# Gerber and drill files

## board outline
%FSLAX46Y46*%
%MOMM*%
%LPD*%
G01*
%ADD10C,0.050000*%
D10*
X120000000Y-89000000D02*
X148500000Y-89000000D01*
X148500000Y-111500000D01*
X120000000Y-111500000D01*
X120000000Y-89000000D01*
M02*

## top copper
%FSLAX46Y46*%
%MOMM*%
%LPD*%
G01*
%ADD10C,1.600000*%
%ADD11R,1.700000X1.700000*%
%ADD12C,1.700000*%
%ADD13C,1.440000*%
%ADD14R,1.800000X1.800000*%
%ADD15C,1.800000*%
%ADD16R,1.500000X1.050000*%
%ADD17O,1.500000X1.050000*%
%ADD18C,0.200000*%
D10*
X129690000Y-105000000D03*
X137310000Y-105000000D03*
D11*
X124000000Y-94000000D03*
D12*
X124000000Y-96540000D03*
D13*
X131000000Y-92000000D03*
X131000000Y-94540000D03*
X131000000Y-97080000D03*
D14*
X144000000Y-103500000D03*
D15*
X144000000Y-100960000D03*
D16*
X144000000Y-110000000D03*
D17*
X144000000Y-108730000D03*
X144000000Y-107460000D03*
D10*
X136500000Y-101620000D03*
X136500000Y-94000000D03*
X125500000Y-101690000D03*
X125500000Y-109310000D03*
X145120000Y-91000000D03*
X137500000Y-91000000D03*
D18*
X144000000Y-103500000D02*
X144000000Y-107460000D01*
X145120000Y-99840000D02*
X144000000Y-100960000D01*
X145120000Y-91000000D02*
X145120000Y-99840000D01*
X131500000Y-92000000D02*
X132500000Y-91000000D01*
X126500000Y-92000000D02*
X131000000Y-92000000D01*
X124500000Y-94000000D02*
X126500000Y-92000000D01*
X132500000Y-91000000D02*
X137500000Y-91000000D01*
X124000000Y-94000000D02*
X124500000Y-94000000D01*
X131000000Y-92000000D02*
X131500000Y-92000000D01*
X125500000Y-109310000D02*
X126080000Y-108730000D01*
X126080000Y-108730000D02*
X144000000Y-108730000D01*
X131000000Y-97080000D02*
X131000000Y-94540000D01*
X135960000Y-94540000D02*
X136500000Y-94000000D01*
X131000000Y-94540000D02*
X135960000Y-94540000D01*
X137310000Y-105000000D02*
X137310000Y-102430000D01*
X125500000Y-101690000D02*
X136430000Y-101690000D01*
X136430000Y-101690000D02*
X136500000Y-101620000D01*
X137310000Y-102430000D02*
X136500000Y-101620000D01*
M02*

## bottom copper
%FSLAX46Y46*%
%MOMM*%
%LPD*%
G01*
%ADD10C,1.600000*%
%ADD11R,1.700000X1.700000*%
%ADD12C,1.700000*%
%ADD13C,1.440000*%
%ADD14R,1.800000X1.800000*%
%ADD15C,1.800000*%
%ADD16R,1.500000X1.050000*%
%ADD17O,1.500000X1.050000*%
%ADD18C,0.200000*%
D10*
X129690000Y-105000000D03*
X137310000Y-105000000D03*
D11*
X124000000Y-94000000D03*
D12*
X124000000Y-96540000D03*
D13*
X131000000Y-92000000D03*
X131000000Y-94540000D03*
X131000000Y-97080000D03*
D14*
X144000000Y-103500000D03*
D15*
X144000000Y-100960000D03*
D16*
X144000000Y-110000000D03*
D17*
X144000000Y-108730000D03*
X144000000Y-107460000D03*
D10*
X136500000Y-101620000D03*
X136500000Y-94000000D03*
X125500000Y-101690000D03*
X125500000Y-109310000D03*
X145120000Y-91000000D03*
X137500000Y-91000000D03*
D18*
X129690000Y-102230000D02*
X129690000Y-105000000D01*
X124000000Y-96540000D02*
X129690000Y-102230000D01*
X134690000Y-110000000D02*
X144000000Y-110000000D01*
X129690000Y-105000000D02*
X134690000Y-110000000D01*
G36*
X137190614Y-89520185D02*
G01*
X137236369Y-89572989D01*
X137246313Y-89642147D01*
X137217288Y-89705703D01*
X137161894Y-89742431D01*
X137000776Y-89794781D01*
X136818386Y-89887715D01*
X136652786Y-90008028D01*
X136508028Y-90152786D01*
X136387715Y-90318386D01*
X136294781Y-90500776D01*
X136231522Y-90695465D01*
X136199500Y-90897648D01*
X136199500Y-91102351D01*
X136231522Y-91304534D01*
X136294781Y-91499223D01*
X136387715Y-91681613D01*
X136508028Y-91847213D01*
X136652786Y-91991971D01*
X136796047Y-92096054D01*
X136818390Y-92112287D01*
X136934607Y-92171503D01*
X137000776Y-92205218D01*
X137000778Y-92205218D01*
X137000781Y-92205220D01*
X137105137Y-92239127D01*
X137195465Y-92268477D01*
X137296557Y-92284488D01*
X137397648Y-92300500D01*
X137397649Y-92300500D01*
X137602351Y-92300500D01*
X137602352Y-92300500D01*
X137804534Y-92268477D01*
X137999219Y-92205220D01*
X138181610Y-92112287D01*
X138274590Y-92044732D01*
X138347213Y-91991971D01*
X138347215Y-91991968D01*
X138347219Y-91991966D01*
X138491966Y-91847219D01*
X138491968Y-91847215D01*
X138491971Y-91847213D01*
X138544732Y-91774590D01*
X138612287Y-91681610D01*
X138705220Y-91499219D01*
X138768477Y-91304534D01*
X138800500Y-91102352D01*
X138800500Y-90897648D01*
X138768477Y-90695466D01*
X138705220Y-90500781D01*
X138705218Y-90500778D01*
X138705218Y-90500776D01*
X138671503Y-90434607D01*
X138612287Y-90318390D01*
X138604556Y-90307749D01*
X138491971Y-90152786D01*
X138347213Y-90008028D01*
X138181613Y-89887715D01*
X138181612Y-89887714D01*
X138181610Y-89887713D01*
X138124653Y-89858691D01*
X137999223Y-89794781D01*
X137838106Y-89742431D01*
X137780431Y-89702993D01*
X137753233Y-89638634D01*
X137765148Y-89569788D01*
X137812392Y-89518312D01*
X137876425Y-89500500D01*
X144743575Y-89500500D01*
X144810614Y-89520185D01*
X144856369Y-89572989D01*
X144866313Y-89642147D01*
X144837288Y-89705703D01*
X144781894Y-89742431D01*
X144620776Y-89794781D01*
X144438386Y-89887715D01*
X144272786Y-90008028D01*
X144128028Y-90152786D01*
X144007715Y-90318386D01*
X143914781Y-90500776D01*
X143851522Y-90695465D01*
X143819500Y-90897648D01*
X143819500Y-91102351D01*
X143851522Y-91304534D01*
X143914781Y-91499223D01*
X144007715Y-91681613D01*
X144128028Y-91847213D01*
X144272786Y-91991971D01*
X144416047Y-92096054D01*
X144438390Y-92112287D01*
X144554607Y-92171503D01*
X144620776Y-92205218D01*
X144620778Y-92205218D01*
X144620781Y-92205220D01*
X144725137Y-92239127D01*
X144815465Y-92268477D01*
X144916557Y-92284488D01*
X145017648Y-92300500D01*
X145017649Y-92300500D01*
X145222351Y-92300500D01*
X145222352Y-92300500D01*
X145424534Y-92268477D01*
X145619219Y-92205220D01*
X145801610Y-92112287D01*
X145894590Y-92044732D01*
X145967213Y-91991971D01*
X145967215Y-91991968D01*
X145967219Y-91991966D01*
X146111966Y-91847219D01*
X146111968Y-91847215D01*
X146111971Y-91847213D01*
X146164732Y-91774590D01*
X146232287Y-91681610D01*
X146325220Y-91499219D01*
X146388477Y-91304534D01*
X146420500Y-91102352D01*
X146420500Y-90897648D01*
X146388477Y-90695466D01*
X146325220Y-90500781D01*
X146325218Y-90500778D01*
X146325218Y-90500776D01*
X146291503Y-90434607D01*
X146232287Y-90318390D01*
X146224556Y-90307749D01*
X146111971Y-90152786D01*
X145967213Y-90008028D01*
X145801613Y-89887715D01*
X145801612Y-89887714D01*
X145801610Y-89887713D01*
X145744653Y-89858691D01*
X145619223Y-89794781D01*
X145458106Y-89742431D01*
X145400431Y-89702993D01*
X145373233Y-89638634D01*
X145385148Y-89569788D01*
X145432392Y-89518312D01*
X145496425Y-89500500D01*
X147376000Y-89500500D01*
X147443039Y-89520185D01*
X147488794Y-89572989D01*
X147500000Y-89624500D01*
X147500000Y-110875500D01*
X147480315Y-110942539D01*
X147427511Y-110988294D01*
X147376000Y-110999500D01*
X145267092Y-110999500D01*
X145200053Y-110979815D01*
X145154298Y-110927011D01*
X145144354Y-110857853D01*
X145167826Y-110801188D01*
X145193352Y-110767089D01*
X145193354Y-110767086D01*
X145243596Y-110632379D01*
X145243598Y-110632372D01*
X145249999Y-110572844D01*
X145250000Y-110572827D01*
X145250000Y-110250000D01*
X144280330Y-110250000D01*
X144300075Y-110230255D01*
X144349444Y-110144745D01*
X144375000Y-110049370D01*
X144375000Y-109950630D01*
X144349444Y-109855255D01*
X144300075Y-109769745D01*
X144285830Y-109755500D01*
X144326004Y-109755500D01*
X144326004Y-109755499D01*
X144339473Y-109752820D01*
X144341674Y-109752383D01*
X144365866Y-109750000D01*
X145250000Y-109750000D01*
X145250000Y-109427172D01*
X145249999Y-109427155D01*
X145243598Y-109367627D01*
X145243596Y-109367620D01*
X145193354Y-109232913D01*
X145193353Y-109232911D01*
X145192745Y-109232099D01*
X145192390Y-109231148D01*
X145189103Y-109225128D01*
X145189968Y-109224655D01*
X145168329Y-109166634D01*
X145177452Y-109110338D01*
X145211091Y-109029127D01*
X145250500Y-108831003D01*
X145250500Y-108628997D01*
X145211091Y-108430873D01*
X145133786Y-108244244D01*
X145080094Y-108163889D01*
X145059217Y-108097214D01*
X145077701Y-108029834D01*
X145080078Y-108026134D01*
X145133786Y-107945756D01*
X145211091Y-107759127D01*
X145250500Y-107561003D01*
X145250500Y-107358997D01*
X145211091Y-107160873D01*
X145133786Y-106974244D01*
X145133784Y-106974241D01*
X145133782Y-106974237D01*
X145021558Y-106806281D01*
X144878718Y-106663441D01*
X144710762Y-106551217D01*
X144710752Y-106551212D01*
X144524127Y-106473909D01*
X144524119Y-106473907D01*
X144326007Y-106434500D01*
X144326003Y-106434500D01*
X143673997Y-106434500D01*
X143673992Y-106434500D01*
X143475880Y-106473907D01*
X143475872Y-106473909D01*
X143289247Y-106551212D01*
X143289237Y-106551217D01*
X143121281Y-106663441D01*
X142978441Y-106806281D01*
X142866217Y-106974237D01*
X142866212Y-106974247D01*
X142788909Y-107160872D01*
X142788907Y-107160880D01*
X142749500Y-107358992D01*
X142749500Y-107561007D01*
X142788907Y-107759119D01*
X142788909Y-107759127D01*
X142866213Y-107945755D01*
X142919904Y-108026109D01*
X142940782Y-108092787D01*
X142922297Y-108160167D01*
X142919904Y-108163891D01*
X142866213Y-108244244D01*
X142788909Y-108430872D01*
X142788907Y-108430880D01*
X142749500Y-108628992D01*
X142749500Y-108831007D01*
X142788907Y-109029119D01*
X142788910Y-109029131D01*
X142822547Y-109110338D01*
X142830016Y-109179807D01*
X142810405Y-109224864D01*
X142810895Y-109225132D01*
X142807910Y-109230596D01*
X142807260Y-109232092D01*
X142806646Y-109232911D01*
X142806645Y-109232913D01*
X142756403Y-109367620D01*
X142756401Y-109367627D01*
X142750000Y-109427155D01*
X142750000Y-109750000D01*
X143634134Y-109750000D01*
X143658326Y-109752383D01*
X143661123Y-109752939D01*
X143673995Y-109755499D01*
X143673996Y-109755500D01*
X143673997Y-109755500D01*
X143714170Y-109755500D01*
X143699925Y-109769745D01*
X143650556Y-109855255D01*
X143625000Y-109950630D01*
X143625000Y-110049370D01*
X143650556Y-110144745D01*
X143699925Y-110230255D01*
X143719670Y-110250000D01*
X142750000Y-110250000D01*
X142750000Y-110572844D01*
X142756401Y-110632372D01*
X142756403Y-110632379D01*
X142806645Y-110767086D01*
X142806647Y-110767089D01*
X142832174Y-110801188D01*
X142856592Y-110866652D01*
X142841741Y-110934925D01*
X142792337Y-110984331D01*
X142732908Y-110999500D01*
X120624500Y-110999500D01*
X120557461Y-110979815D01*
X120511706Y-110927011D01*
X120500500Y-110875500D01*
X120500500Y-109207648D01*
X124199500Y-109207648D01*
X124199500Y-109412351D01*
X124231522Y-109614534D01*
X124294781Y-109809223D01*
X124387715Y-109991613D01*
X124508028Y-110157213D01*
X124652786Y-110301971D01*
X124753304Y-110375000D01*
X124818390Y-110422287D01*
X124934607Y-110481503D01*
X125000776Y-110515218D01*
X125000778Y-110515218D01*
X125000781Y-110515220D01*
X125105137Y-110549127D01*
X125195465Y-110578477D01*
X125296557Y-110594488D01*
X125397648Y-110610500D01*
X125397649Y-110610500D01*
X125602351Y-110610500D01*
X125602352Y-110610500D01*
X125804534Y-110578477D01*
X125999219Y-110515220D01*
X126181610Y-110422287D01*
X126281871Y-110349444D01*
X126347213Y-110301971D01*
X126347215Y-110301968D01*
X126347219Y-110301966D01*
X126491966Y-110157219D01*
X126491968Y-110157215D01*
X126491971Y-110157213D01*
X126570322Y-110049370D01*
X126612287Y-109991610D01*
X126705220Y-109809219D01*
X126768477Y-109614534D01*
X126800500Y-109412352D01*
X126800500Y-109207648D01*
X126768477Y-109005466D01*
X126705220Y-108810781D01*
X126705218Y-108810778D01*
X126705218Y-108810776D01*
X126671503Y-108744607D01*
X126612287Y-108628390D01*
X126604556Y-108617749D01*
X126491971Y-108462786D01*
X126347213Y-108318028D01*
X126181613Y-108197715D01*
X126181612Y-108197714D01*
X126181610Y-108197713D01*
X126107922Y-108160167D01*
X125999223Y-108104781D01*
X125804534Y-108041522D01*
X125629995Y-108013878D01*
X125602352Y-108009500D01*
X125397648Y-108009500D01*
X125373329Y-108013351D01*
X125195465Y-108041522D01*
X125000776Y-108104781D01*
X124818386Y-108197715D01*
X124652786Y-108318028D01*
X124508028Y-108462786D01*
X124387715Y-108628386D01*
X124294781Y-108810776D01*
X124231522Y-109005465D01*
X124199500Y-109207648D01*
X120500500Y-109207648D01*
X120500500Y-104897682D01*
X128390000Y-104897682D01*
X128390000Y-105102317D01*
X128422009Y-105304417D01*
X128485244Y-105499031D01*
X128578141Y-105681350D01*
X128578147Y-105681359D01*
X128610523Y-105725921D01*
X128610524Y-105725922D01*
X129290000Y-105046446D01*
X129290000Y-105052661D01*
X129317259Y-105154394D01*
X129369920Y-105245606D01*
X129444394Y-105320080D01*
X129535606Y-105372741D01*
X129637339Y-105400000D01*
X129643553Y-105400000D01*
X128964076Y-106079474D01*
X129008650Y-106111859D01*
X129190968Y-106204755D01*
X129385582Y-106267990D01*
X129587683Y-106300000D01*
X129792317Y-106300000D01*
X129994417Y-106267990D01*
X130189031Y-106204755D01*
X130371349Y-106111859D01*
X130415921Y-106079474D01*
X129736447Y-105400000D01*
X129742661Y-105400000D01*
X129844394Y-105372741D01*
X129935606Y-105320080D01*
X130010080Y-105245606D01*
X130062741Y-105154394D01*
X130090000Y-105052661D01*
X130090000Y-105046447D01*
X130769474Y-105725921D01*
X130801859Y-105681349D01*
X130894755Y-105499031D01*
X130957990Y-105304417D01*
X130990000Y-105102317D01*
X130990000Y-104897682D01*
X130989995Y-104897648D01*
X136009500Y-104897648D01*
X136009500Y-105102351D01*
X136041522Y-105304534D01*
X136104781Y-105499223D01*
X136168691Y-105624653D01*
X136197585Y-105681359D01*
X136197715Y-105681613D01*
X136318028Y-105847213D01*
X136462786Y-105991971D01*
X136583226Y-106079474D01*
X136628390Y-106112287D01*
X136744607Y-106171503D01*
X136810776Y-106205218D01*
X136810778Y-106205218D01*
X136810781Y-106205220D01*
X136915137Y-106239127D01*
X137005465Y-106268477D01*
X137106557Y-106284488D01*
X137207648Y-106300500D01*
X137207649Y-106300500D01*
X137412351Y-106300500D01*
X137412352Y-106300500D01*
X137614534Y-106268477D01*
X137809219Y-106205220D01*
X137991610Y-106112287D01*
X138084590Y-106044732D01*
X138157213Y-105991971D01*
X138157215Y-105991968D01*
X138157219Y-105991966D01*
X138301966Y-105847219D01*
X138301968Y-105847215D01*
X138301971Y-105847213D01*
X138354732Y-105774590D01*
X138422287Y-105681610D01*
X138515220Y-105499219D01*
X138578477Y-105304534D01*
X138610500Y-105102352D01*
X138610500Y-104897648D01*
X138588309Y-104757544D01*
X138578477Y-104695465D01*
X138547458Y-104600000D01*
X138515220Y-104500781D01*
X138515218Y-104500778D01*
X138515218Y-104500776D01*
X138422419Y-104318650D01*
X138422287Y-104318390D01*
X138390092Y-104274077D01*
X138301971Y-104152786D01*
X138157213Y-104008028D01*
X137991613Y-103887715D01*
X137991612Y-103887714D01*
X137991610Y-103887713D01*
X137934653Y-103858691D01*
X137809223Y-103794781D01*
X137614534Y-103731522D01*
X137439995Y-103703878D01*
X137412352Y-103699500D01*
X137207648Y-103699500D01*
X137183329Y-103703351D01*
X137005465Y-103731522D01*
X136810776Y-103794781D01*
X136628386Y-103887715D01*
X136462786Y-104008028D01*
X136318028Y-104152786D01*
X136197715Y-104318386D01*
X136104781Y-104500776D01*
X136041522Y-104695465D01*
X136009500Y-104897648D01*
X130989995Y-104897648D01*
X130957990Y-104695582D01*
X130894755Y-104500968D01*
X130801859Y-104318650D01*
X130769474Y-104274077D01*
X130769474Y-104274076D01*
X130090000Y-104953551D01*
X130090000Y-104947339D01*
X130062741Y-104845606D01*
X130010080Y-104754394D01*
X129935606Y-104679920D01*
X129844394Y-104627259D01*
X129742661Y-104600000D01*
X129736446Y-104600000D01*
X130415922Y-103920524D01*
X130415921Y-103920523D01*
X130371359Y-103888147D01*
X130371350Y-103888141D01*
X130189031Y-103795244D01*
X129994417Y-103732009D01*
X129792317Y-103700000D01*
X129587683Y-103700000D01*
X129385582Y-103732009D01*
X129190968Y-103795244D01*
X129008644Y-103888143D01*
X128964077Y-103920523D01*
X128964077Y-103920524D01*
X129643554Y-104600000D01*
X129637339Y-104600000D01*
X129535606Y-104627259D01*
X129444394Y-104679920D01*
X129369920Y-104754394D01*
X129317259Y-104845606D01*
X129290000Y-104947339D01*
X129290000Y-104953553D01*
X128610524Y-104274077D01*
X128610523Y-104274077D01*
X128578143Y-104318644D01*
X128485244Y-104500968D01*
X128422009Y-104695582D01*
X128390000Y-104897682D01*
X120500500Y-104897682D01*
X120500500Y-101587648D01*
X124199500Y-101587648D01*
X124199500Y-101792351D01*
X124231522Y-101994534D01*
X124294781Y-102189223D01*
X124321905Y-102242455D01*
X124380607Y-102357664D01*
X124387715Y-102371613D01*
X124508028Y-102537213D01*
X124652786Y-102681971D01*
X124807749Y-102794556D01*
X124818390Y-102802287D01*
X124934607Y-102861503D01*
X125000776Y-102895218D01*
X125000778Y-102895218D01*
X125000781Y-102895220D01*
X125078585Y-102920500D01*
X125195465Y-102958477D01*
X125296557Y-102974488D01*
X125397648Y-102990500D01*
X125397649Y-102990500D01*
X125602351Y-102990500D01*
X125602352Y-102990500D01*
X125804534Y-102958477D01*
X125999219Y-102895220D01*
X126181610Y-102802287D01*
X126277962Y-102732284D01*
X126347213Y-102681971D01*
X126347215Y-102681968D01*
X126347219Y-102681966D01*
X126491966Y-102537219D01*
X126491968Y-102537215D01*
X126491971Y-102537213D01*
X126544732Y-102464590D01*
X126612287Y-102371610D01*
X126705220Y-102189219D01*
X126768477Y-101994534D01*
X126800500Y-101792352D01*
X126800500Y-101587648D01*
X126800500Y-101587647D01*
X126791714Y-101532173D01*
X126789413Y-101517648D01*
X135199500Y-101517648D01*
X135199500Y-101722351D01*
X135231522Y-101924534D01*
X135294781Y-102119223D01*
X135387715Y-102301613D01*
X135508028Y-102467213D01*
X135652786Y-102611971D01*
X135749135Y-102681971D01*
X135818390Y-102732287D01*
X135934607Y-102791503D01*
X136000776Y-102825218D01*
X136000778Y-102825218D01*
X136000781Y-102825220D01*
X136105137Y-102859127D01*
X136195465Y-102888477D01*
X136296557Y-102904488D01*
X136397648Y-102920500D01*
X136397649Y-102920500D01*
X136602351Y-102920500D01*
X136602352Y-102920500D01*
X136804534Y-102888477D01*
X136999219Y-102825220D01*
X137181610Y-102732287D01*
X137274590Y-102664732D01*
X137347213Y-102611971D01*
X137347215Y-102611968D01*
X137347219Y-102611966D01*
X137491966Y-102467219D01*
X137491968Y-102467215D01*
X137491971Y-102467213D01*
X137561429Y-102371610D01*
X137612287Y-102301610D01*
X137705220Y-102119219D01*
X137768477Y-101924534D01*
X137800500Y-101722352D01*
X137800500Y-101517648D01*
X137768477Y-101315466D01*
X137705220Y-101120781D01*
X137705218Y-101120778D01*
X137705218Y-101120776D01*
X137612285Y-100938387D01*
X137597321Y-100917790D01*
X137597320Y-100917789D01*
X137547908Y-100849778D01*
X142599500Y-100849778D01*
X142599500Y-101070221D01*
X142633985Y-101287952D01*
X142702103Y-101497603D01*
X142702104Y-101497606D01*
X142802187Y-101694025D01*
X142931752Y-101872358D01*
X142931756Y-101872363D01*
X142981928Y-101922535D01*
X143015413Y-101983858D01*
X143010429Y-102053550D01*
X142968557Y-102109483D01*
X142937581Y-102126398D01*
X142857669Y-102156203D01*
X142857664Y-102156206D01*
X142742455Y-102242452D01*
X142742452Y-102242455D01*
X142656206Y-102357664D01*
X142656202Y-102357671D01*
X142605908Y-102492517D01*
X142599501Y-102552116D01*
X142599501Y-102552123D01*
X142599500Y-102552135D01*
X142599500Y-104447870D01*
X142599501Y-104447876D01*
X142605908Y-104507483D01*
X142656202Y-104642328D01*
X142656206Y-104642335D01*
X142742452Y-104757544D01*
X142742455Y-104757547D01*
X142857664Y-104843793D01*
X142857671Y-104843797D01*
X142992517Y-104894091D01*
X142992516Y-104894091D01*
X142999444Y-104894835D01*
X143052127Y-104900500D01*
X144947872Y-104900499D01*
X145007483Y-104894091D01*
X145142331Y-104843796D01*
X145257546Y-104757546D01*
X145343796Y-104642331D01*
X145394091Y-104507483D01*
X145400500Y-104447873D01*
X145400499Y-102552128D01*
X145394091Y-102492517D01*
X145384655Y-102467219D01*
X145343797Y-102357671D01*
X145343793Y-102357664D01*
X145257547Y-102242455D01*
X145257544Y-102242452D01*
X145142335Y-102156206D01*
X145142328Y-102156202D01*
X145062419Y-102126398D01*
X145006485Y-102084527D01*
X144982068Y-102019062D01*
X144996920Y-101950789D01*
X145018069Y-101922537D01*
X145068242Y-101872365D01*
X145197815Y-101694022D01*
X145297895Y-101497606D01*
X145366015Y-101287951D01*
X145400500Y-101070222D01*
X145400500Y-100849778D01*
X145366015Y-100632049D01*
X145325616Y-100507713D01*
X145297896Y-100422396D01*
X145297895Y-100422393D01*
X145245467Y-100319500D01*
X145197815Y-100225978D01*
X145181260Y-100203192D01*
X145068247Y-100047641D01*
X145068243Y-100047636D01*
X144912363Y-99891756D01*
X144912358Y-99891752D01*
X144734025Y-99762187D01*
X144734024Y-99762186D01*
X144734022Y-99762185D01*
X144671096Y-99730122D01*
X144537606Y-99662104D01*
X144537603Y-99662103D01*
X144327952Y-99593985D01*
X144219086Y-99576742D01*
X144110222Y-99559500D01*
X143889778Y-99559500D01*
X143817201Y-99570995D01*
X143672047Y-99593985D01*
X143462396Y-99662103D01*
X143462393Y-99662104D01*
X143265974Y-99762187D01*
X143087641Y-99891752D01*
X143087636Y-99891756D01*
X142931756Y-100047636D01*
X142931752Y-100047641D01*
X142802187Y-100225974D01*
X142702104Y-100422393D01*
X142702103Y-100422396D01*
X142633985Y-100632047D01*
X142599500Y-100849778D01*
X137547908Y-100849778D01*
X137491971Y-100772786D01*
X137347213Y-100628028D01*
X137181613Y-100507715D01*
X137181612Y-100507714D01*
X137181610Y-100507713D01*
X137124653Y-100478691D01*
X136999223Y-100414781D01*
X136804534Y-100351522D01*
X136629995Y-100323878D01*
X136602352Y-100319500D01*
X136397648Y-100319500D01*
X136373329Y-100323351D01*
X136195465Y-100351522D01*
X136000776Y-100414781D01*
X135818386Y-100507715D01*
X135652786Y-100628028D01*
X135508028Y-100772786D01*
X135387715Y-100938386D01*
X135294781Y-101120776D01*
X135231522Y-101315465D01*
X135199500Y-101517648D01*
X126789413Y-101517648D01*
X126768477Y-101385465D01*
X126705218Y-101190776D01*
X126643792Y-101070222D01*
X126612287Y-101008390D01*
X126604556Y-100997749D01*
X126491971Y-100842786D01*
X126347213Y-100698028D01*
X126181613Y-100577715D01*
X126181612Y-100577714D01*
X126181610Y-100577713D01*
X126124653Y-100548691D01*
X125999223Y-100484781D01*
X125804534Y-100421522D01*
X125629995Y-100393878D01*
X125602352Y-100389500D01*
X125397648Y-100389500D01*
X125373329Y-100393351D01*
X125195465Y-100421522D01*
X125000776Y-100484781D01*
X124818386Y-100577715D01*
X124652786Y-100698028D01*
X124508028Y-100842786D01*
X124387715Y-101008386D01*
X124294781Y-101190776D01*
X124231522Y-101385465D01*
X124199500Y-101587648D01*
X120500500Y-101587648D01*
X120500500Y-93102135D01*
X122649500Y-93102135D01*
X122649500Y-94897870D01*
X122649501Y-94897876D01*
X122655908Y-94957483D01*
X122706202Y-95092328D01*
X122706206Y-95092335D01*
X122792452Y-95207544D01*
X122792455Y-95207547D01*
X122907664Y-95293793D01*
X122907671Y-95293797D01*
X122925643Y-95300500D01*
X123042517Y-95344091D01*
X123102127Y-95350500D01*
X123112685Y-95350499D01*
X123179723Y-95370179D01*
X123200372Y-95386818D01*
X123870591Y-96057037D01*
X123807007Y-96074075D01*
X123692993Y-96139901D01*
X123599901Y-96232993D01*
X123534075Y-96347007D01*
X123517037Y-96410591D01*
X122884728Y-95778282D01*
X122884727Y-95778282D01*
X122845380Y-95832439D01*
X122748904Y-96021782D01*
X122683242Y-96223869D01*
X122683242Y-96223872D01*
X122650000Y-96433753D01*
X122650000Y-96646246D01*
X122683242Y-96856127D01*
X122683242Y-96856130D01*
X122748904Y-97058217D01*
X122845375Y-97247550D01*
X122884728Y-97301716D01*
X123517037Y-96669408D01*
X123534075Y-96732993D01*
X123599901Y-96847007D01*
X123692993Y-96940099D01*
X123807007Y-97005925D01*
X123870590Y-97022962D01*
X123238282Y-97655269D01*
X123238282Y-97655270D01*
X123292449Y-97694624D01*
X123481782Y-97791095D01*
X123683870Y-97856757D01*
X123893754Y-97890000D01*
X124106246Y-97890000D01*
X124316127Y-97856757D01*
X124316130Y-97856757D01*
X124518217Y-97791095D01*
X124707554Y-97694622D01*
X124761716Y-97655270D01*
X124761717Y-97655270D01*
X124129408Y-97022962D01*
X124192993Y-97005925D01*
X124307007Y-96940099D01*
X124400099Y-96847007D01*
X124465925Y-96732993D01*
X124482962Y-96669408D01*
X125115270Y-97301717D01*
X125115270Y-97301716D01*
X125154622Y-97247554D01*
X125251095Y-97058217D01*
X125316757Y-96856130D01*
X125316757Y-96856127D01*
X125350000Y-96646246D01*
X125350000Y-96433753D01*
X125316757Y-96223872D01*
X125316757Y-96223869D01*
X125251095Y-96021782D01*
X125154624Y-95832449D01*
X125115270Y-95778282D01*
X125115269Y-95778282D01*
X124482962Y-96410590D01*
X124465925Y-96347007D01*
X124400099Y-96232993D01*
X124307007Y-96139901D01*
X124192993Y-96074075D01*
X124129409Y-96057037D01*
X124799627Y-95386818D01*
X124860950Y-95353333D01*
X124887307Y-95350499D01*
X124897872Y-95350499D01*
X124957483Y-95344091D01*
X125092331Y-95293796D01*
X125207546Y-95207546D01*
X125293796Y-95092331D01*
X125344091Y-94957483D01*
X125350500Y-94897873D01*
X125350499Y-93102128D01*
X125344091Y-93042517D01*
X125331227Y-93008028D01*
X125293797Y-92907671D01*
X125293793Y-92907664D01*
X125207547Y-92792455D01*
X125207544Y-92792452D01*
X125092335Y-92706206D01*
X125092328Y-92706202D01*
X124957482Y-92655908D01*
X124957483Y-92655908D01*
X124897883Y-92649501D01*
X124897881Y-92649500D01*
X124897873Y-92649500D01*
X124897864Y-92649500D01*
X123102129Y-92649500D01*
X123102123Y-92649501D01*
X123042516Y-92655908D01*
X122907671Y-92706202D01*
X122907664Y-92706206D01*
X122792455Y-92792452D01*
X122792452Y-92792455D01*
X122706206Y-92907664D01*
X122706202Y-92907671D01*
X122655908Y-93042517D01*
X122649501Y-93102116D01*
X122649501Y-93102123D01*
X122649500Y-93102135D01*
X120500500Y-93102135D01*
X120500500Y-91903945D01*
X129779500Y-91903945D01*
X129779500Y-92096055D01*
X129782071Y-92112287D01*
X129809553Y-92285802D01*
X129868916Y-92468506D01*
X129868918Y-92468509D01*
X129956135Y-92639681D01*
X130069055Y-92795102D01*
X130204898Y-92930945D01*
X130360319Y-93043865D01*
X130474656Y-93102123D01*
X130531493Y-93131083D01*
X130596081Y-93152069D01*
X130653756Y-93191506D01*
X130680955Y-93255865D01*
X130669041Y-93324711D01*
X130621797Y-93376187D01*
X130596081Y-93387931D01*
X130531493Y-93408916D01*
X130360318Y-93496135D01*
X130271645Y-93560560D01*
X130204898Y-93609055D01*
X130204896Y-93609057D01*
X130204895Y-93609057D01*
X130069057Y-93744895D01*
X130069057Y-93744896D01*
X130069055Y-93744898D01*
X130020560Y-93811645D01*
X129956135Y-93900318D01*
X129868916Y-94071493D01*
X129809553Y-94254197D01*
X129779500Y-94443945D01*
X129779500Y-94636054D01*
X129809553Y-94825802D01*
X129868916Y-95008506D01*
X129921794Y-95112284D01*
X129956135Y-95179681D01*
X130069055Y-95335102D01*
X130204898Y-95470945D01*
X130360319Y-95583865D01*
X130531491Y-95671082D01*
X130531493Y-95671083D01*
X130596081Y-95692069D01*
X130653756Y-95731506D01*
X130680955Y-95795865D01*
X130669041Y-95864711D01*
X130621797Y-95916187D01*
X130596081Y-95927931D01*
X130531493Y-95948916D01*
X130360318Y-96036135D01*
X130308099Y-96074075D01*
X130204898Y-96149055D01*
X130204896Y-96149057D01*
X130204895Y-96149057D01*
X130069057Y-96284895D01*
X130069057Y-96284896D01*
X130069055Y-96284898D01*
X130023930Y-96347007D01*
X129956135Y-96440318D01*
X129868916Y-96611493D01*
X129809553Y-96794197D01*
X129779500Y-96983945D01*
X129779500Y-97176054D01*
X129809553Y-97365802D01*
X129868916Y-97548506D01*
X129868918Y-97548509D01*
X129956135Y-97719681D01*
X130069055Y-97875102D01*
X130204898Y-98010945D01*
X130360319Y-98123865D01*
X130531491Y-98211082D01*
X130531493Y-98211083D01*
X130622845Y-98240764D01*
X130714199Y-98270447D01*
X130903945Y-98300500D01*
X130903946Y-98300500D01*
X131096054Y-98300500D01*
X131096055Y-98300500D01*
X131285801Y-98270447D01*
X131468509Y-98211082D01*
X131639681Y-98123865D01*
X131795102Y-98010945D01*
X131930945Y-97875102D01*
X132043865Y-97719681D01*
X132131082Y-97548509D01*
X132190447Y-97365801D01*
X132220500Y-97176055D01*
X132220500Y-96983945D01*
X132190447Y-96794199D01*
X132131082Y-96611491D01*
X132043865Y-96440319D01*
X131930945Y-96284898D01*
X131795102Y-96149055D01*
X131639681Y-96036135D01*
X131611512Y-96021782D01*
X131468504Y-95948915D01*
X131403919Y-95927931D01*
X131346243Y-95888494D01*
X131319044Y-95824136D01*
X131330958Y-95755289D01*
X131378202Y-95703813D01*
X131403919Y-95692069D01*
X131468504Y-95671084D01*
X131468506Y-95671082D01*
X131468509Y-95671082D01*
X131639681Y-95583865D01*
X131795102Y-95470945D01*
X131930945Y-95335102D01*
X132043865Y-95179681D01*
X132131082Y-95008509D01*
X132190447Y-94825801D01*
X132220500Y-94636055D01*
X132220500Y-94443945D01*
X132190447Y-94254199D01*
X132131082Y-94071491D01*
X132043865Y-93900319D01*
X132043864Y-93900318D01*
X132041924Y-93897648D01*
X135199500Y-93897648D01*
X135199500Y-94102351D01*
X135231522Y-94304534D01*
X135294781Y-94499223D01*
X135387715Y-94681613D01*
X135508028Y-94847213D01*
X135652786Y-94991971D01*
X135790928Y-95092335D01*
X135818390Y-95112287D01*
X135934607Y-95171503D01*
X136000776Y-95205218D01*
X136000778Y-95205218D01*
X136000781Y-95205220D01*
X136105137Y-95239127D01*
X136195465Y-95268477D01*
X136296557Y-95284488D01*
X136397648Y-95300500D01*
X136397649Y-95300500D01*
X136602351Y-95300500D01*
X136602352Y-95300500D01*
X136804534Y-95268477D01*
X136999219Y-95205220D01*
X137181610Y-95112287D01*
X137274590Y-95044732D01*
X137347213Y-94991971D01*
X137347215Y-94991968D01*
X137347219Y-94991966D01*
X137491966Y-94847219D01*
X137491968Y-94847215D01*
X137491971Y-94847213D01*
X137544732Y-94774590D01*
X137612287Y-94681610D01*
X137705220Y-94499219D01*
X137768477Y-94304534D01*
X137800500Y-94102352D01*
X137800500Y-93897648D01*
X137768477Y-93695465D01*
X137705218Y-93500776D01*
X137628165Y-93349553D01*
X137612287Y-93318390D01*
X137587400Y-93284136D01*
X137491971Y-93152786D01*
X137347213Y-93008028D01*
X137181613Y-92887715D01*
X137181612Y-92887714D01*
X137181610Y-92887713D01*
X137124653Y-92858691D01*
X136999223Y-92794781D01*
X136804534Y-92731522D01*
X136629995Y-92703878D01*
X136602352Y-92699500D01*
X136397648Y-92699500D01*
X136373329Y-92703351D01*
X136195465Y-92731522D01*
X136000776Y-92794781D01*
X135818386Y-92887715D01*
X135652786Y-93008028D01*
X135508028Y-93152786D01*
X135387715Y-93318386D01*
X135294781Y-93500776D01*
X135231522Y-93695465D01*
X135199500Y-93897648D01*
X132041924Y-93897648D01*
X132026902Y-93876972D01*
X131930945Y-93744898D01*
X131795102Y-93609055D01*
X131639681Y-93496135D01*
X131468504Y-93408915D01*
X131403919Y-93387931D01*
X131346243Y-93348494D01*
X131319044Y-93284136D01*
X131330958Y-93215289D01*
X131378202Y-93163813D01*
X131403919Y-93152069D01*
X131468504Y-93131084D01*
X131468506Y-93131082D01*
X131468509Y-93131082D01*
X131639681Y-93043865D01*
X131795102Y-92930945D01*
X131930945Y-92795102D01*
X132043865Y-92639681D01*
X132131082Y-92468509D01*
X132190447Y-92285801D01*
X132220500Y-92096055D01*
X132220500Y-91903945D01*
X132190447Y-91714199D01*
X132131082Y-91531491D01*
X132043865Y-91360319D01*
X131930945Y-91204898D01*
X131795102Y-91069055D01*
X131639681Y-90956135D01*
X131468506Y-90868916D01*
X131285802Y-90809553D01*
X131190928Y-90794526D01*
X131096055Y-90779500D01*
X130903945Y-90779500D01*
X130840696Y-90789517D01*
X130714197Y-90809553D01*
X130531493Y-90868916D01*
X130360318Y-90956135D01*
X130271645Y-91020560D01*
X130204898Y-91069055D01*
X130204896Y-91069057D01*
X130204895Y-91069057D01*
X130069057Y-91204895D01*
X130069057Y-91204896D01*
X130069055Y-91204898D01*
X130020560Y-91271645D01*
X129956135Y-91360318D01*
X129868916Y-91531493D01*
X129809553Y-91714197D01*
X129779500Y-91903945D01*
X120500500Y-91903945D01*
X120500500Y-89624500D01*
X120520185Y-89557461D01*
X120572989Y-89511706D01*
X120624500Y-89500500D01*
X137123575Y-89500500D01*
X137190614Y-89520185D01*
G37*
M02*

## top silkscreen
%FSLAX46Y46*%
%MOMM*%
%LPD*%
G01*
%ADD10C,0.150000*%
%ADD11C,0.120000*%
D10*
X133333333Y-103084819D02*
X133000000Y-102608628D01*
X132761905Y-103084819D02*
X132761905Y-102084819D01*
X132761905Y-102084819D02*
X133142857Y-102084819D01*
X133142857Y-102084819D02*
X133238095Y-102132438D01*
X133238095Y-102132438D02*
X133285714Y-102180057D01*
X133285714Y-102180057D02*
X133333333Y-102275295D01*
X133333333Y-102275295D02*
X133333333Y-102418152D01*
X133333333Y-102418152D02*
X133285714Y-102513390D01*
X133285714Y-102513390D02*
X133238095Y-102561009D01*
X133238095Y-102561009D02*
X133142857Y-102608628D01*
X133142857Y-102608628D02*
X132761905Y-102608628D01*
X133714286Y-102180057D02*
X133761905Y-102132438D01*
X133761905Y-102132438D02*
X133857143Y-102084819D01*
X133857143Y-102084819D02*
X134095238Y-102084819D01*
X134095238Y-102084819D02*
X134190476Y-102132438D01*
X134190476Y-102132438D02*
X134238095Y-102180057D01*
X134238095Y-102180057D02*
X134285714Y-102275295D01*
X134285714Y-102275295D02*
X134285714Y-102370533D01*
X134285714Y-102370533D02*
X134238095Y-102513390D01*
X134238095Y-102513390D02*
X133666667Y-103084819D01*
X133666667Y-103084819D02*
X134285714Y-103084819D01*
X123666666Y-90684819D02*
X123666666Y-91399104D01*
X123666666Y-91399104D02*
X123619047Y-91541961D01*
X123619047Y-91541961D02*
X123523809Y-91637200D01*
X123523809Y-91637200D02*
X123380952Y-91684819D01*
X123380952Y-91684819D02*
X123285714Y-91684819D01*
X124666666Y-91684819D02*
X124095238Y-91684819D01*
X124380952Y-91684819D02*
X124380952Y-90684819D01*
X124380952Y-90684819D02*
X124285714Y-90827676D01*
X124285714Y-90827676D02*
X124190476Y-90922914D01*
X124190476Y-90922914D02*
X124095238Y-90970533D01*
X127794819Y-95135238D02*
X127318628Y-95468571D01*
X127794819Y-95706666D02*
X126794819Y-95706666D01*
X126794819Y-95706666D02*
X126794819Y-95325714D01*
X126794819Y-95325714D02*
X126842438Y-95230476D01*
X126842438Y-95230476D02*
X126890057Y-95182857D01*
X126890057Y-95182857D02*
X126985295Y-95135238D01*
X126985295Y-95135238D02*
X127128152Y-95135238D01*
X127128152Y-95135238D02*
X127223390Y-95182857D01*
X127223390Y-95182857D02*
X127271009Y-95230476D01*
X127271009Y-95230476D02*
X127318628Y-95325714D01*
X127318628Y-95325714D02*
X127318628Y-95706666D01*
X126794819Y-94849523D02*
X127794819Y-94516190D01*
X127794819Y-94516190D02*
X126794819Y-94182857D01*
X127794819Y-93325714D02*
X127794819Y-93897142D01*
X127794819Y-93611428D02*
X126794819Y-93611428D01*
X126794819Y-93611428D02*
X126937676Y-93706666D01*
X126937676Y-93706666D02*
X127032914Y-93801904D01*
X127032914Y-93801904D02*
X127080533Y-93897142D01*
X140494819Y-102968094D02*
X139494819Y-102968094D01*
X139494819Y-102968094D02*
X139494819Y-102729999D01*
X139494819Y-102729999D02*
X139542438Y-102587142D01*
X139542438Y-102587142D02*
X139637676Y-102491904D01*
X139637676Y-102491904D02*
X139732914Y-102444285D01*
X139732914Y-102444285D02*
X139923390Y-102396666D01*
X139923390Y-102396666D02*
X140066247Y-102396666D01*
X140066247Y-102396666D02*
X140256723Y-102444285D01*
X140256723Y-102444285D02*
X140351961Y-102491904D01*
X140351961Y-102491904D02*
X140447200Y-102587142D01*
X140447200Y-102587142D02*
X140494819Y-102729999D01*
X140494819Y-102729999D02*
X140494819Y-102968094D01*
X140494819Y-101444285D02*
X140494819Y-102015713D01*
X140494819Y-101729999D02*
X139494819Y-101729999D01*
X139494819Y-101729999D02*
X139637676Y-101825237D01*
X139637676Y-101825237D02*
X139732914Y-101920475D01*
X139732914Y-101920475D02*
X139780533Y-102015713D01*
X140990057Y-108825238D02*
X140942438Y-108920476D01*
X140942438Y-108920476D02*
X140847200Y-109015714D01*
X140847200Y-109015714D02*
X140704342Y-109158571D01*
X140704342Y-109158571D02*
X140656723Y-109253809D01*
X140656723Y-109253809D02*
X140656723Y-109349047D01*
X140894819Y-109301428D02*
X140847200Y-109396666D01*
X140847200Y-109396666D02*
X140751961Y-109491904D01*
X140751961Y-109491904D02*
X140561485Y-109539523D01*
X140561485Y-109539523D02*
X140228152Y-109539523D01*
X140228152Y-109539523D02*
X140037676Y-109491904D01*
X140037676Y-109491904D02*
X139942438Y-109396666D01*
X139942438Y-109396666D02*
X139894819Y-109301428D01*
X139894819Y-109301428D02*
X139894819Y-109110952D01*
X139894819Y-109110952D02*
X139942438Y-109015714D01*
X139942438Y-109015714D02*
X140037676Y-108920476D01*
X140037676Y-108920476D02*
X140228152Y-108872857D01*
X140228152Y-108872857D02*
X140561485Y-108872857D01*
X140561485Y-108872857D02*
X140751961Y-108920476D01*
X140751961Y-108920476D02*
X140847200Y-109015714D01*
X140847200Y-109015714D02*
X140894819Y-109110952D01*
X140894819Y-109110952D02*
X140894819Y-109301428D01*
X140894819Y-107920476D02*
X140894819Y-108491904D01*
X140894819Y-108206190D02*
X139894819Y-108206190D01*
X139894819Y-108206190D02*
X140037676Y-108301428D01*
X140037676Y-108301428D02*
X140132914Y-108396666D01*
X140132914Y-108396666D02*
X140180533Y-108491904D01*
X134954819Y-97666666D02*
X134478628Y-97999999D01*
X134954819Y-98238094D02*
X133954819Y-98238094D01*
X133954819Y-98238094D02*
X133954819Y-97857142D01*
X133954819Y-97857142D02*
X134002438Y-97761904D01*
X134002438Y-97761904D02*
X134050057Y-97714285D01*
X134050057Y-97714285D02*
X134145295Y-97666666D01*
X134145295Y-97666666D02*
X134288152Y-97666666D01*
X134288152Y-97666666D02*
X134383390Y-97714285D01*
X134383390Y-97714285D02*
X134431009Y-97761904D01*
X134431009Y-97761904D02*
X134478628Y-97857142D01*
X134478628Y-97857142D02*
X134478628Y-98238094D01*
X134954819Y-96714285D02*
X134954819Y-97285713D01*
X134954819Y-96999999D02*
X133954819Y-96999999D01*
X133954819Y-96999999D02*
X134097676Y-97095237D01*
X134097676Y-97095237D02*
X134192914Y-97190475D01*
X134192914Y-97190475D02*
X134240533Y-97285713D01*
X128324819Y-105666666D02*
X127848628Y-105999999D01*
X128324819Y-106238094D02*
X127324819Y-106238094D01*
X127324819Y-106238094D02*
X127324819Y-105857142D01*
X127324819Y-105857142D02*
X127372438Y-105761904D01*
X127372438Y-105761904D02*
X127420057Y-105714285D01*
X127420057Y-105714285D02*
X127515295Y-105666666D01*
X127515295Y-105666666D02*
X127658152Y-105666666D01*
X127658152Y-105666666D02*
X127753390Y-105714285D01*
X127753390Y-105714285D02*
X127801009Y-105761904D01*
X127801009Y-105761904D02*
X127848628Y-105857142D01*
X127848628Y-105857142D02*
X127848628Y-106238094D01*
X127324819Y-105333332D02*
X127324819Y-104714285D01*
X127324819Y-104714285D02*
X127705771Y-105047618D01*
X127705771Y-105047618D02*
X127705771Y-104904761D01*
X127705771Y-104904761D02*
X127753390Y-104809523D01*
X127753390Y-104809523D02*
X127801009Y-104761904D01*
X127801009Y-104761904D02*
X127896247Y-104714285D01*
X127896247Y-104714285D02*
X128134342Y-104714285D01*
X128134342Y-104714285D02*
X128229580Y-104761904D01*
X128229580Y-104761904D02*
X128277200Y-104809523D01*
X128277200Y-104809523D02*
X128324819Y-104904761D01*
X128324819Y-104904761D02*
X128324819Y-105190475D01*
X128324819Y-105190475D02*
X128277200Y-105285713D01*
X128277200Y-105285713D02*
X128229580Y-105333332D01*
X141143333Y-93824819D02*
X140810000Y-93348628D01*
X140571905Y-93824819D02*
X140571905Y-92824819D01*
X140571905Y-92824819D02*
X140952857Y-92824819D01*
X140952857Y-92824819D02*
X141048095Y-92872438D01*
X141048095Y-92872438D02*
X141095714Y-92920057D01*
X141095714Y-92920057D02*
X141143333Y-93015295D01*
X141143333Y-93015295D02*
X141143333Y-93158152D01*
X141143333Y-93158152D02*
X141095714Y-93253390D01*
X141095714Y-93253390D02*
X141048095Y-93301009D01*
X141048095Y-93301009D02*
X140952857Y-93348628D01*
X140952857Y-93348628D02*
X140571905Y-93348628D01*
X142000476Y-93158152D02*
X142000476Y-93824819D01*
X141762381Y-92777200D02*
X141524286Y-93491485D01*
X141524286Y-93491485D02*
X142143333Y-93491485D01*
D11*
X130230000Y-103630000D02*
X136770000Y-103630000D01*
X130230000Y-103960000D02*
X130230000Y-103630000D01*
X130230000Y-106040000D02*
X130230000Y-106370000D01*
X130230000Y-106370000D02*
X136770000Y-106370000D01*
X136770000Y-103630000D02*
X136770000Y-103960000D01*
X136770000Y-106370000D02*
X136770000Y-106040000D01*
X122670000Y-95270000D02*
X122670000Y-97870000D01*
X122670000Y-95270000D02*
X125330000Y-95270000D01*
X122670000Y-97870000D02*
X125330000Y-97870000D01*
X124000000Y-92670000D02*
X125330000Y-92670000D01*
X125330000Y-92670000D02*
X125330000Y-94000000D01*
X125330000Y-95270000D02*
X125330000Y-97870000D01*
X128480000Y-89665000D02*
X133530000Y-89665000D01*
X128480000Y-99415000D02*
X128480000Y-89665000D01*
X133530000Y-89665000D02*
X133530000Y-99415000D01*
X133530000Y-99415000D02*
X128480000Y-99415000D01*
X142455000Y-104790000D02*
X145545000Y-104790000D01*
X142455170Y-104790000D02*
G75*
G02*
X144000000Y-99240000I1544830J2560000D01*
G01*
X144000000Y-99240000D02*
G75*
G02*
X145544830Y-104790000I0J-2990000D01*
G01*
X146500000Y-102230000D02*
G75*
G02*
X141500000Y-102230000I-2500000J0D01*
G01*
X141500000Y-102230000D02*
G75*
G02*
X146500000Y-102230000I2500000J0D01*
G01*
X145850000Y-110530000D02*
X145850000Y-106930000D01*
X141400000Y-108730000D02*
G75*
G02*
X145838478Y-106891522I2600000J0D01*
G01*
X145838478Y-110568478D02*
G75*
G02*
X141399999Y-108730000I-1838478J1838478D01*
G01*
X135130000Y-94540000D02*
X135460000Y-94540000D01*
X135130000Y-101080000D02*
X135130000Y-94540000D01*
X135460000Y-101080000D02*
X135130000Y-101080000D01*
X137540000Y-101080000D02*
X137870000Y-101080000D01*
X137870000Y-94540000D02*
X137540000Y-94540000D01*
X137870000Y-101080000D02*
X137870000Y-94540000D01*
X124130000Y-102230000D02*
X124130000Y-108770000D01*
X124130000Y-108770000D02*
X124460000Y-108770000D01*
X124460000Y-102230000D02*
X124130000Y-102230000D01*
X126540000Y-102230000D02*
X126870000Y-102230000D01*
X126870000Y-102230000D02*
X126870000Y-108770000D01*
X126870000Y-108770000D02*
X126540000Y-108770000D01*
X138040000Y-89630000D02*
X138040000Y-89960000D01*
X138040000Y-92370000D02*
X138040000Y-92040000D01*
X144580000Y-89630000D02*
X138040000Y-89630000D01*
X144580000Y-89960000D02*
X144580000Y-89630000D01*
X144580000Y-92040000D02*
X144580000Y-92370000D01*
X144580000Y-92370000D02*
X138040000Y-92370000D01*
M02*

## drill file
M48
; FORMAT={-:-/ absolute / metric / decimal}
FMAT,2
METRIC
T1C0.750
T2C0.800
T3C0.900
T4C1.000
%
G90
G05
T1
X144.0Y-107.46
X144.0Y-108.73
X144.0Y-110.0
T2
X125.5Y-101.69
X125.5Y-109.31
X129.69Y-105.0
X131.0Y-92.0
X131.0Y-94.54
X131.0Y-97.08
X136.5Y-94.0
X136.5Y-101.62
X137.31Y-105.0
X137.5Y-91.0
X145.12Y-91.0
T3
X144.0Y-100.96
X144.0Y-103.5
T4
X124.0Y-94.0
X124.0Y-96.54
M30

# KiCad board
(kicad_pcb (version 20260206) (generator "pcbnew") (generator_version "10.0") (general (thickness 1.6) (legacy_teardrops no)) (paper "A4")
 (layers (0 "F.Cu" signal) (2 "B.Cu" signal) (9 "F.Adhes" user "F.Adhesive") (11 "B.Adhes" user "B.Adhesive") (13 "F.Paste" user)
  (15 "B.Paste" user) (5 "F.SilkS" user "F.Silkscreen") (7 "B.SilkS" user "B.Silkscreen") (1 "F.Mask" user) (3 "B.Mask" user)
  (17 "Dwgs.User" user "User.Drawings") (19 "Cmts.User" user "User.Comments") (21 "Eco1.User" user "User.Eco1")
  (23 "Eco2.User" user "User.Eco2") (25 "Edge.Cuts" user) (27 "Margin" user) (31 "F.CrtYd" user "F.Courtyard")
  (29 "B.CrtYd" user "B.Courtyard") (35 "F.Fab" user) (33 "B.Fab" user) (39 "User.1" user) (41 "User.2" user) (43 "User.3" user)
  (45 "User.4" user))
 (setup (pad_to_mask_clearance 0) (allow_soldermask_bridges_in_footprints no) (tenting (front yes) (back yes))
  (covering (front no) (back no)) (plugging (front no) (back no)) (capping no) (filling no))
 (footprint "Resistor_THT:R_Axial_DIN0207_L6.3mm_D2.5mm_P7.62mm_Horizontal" (layer "F.Cu") (at 129.69 105)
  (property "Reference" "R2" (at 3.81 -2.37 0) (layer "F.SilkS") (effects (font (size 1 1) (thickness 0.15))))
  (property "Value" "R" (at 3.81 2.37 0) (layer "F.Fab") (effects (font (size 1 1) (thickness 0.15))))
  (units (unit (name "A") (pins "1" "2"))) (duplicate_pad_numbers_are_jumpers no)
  (fp_line (start 0.54 -1.37) (end 7.08 -1.37) (stroke (width 0.12) (type solid)) (layer "F.SilkS"))
  (fp_line (start 0.54 -1.04) (end 0.54 -1.37) (stroke (width 0.12) (type solid)) (layer "F.SilkS"))
  (fp_line (start 0.54 1.04) (end 0.54 1.37) (stroke (width 0.12) (type solid)) (layer "F.SilkS"))
  (fp_line (start 0.54 1.37) (end 7.08 1.37) (stroke (width 0.12) (type solid)) (layer "F.SilkS"))
  (fp_line (start 7.08 -1.37) (end 7.08 -1.04) (stroke (width 0.12) (type solid)) (layer "F.SilkS"))
  (fp_line (start 7.08 1.37) (end 7.08 1.04) (stroke (width 0.12) (type solid)) (layer "F.SilkS"))
  (pad "1" thru_hole circle (at 0 0) (size 1.6 1.6) (drill 0.8) (layers "*.Cu" "*.Mask") (remove_unused_layers no) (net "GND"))
  (pad "2" thru_hole circle (at 7.62 0) (size 1.6 1.6) (drill 0.8) (layers "*.Cu" "*.Mask") (remove_unused_layers no) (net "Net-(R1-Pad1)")))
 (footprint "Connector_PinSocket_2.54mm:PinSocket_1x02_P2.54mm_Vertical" (layer "F.Cu") (at 124 94)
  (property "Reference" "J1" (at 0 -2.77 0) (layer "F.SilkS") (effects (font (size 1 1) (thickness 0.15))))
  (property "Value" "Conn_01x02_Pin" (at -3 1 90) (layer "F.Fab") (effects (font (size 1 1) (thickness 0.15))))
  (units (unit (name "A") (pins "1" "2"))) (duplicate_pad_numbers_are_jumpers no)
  (fp_line (start -1.33 1.27) (end -1.33 3.87) (stroke (width 0.12) (type solid)) (layer "F.SilkS"))
  (fp_line (start -1.33 1.27) (end 1.33 1.27) (stroke (width 0.12) (type solid)) (layer "F.SilkS"))
  (fp_line (start -1.33 3.87) (end 1.33 3.87) (stroke (width 0.12) (type solid)) (layer "F.SilkS"))
  (fp_line (start 0 -1.33) (end 1.33 -1.33) (stroke (width 0.12) (type solid)) (layer "F.SilkS"))
  (fp_line (start 1.33 -1.33) (end 1.33 0) (stroke (width 0.12) (type solid)) (layer "F.SilkS"))
  (fp_line (start 1.33 1.27) (end 1.33 3.87) (stroke (width 0.12) (type solid)) (layer "F.SilkS"))
  (pad "1" thru_hole rect (at 0 0) (size 1.7 1.7) (drill 1) (layers "*.Cu" "*.Mask") (remove_unused_layers no) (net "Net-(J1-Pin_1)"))
  (pad "2" thru_hole circle (at 0 2.54) (size 1.7 1.7) (drill 1) (layers "*.Cu" "*.Mask") (remove_unused_layers no) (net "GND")))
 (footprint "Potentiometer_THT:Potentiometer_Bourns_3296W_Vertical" (layer "F.Cu") (at 131 92 90)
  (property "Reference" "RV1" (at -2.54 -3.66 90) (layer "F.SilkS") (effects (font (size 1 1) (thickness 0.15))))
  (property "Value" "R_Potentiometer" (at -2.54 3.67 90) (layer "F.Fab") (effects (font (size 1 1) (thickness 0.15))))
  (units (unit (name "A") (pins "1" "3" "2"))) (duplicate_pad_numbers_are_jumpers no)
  (fp_line (start 2.335 -2.52) (end 2.335 2.53) (stroke (width 0.12) (type solid)) (layer "F.SilkS"))
  (fp_line (start -7.415 -2.52) (end 2.335 -2.52) (stroke (width 0.12) (type solid)) (layer "F.SilkS"))
  (fp_line (start 2.335 2.53) (end -7.415 2.53) (stroke (width 0.12) (type solid)) (layer "F.SilkS"))
  (fp_line (start -7.415 2.53) (end -7.415 -2.52) (stroke (width 0.12) (type solid)) (layer "F.SilkS"))
  (pad "1" thru_hole circle (at 0 0 90) (size 1.44 1.44) (drill 0.8) (layers "*.Cu" "*.Mask") (remove_unused_layers no)
   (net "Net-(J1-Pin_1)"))
  (pad "2" thru_hole circle (at -2.54 0 90) (size 1.44 1.44) (drill 0.8) (layers "*.Cu" "*.Mask") (remove_unused_layers no)
   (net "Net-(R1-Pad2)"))
  (pad "3" thru_hole circle (at -5.08 0 90) (size 1.44 1.44) (drill 0.8) (layers "*.Cu" "*.Mask") (remove_unused_layers no)
   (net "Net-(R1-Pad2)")))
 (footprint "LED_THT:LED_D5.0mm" (layer "F.Cu") (at 144 103.5 90)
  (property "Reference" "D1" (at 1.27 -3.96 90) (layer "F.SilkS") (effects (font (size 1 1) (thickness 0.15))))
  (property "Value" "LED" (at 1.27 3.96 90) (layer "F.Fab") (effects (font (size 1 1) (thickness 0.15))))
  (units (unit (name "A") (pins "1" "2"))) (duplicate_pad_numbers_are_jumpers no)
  (fp_line (start -1.29 -1.545) (end -1.29 1.545) (stroke (width 0.12) (type solid)) (layer "F.SilkS"))
  (fp_arc (start -1.29 -1.54483) (mid 2.071779 -2.880495) (end 4.26 0) (stroke (width 0.12) (type solid)) (layer "F.SilkS"))
  (fp_arc (start 4.26 0) (mid 2.071779 2.880495) (end -1.29 1.54483) (stroke (width 0.12) (type solid)) (layer "F.SilkS"))
  (fp_circle (center 1.27 0) (end 3.77 0) (stroke (width 0.12) (type solid)) (fill no) (layer "F.SilkS"))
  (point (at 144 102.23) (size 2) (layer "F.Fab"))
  (pad "1" thru_hole rect (at 0 0 90) (size 1.8 1.8) (drill 0.9) (layers "*.Cu" "*.Mask") (remove_unused_layers no) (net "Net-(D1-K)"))
  (pad "2" thru_hole circle (at 2.54 0 90) (size 1.8 1.8) (drill 0.9) (layers "*.Cu" "*.Mask") (remove_unused_layers no) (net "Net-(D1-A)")))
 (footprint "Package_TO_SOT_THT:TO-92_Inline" (layer "F.Cu") (at 144 110 90)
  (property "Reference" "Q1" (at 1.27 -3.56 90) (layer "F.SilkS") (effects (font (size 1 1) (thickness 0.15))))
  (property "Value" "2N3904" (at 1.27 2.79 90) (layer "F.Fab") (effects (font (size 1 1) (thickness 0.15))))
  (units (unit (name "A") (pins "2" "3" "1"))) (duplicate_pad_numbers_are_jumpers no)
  (fp_line (start -0.53 1.85) (end 3.07 1.85) (stroke (width 0.12) (type solid)) (layer "F.SilkS"))
  (fp_arc (start 1.27 -2.6) (mid 3.672087 -0.994977) (end 3.108478 1.838478) (stroke (width 0.12) (type solid)) (layer "F.SilkS"))
  (fp_arc (start -0.568478 1.838478) (mid -1.132087 -0.994977) (end 1.27 -2.6) (stroke (width 0.12) (type solid)) (layer "F.SilkS"))
  (pad "1" thru_hole rect (at 0 0 90) (size 1.05 1.5) (drill 0.75) (layers "*.Cu" "*.Mask") (remove_unused_layers no) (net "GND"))
  (pad "2" thru_hole oval (at 1.27 0 90) (size 1.05 1.5) (drill 0.75) (layers "*.Cu" "*.Mask") (remove_unused_layers no) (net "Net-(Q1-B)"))
  (pad "3" thru_hole oval (at 2.54 0 90) (size 1.05 1.5) (drill 0.75) (layers "*.Cu" "*.Mask") (remove_unused_layers no) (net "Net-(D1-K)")))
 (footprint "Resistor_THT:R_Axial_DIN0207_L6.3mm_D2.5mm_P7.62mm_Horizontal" (layer "F.Cu") (at 136.5 101.62 90)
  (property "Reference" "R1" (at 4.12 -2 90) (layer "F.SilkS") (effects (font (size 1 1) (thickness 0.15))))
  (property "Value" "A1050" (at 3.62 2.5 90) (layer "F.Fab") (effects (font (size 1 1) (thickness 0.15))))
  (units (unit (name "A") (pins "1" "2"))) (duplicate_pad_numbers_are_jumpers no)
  (fp_line (start 7.08 -1.37) (end 7.08 -1.04) (stroke (width 0.12) (type solid)) (layer "F.SilkS"))
  (fp_line (start 0.54 -1.37) (end 7.08 -1.37) (stroke (width 0.12) (type solid)) (layer "F.SilkS"))
  (fp_line (start 0.54 -1.04) (end 0.54 -1.37) (stroke (width 0.12) (type solid)) (layer "F.SilkS"))
  (fp_line (start 0.54 1.04) (end 0.54 1.37) (stroke (width 0.12) (type solid)) (layer "F.SilkS"))
  (fp_line (start 7.08 1.37) (end 7.08 1.04) (stroke (width 0.12) (type solid)) (layer "F.SilkS"))
  (fp_line (start 0.54 1.37) (end 7.08 1.37) (stroke (width 0.12) (type solid)) (layer "F.SilkS"))
  (pad "1" thru_hole circle (at 0 0 90) (size 1.6 1.6) (drill 0.8) (layers "*.Cu" "*.Mask") (remove_unused_layers no) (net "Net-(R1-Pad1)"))
  (pad "2" thru_hole circle (at 7.62 0 90) (size 1.6 1.6) (drill 0.8) (layers "*.Cu" "*.Mask") (remove_unused_layers no)
   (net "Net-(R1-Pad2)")))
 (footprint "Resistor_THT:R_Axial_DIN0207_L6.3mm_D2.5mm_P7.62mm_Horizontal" (layer "F.Cu") (at 125.5 101.69 -90)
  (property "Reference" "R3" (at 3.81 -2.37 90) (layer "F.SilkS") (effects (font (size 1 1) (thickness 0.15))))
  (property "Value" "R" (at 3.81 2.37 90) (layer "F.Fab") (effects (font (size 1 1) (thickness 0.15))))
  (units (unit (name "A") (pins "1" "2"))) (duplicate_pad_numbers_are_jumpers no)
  (fp_line (start 0.54 1.37) (end 7.08 1.37) (stroke (width 0.12) (type solid)) (layer "F.SilkS"))
  (fp_line (start 7.08 1.37) (end 7.08 1.04) (stroke (width 0.12) (type solid)) (layer "F.SilkS"))
  (fp_line (start 0.54 1.04) (end 0.54 1.37) (stroke (width 0.12) (type solid)) (layer "F.SilkS"))
  (fp_line (start 0.54 -1.04) (end 0.54 -1.37) (stroke (width 0.12) (type solid)) (layer "F.SilkS"))
  (fp_line (start 0.54 -1.37) (end 7.08 -1.37) (stroke (width 0.12) (type solid)) (layer "F.SilkS"))
  (fp_line (start 7.08 -1.37) (end 7.08 -1.04) (stroke (width 0.12) (type solid)) (layer "F.SilkS"))
  (pad "1" thru_hole circle (at 0 0 270) (size 1.6 1.6) (drill 0.8) (layers "*.Cu" "*.Mask") (remove_unused_layers no) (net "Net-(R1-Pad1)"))
  (pad "2" thru_hole circle (at 7.62 0 270) (size 1.6 1.6) (drill 0.8) (layers "*.Cu" "*.Mask") (remove_unused_layers no) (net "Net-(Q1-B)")))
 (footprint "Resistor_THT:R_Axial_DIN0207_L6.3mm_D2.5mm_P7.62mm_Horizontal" (layer "F.Cu") (at 145.12 91 180)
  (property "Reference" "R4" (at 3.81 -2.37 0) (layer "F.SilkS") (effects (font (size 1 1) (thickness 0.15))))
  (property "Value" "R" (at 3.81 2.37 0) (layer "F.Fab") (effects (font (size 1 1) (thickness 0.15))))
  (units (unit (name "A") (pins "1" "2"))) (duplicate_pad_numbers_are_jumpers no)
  (fp_line (start 7.08 1.37) (end 7.08 1.04) (stroke (width 0.12) (type solid)) (layer "F.SilkS"))
  (fp_line (start 7.08 -1.37) (end 7.08 -1.04) (stroke (width 0.12) (type solid)) (layer "F.SilkS"))
  (fp_line (start 0.54 1.37) (end 7.08 1.37) (stroke (width 0.12) (type solid)) (layer "F.SilkS"))
  (fp_line (start 0.54 1.04) (end 0.54 1.37) (stroke (width 0.12) (type solid)) (layer "F.SilkS"))
  (fp_line (start 0.54 -1.04) (end 0.54 -1.37) (stroke (width 0.12) (type solid)) (layer "F.SilkS"))
  (fp_line (start 0.54 -1.37) (end 7.08 -1.37) (stroke (width 0.12) (type solid)) (layer "F.SilkS"))
  (pad "1" thru_hole circle (at 0 0 180) (size 1.6 1.6) (drill 0.8) (layers "*.Cu" "*.Mask") (remove_unused_layers no) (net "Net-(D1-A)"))
  (pad "2" thru_hole circle (at 7.62 0 180) (size 1.6 1.6) (drill 0.8) (layers "*.Cu" "*.Mask") (remove_unused_layers no)
   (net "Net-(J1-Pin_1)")))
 (gr_rect (start 120 89) (end 148.5 111.5) (stroke (width 0.05) (type default)) (fill no) (layer "Edge.Cuts"))
 (segment (start 144 103.5) (end 144 107.46) (width 0.2) (layer "F.Cu") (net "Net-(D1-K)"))
 (segment (start 145.12 99.84) (end 144 100.96) (width 0.2) (layer "F.Cu") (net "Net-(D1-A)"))
 (segment (start 145.12 91) (end 145.12 99.84) (width 0.2) (layer "F.Cu") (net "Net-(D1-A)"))
 (segment (start 129.69 102.23) (end 129.69 105) (width 0.2) (layer "B.Cu") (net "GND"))
 (segment (start 124 96.54) (end 129.69 102.23) (width 0.2) (layer "B.Cu") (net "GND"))
 (segment (start 134.69 110) (end 144 110) (width 0.2) (layer "B.Cu") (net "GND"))
 (segment (start 129.69 105) (end 134.69 110) (width 0.2) (layer "B.Cu") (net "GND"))
 (segment (start 131.5 92) (end 132.5 91) (width 0.2) (layer "F.Cu") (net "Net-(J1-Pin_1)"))
 (segment (start 126.5 92) (end 131 92) (width 0.2) (layer "F.Cu") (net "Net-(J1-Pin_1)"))
 (segment (start 124.5 94) (end 126.5 92) (width 0.2) (layer "F.Cu") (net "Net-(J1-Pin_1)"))
 (segment (start 132.5 91) (end 137.5 91) (width 0.2) (layer "F.Cu") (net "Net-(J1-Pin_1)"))
 (segment (start 124 94) (end 124.5 94) (width 0.2) (layer "F.Cu") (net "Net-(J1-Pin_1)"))
 (segment (start 131 92) (end 131.5 92) (width 0.2) (layer "F.Cu") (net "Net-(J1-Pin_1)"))
 (segment (start 125.5 109.31) (end 126.08 108.73) (width 0.2) (layer "F.Cu") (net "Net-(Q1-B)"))
 (segment (start 126.08 108.73) (end 144 108.73) (width 0.2) (layer "F.Cu") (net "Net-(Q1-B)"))
 (segment (start 131 97.08) (end 131 94.54) (width 0.2) (layer "F.Cu") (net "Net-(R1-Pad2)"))
 (segment (start 135.96 94.54) (end 136.5 94) (width 0.2) (layer "F.Cu") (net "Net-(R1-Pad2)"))
 (segment (start 131 94.54) (end 135.96 94.54) (width 0.2) (layer "F.Cu") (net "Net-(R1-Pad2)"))
 (segment (start 137.31 105) (end 137.31 102.43) (width 0.2) (layer "F.Cu") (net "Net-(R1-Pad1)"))
 (segment (start 125.5 101.69) (end 136.43 101.69) (width 0.2) (layer "F.Cu") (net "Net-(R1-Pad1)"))
 (segment (start 136.43 101.69) (end 136.5 101.62) (width 0.2) (layer "F.Cu") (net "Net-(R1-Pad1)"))
 (segment (start 137.31 102.43) (end 136.5 101.62) (width 0.2) (layer "F.Cu") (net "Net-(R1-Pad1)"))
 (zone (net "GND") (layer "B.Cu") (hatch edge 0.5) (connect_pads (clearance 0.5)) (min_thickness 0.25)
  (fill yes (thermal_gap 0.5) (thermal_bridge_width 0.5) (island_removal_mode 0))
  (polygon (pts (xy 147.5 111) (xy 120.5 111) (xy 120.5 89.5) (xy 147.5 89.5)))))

